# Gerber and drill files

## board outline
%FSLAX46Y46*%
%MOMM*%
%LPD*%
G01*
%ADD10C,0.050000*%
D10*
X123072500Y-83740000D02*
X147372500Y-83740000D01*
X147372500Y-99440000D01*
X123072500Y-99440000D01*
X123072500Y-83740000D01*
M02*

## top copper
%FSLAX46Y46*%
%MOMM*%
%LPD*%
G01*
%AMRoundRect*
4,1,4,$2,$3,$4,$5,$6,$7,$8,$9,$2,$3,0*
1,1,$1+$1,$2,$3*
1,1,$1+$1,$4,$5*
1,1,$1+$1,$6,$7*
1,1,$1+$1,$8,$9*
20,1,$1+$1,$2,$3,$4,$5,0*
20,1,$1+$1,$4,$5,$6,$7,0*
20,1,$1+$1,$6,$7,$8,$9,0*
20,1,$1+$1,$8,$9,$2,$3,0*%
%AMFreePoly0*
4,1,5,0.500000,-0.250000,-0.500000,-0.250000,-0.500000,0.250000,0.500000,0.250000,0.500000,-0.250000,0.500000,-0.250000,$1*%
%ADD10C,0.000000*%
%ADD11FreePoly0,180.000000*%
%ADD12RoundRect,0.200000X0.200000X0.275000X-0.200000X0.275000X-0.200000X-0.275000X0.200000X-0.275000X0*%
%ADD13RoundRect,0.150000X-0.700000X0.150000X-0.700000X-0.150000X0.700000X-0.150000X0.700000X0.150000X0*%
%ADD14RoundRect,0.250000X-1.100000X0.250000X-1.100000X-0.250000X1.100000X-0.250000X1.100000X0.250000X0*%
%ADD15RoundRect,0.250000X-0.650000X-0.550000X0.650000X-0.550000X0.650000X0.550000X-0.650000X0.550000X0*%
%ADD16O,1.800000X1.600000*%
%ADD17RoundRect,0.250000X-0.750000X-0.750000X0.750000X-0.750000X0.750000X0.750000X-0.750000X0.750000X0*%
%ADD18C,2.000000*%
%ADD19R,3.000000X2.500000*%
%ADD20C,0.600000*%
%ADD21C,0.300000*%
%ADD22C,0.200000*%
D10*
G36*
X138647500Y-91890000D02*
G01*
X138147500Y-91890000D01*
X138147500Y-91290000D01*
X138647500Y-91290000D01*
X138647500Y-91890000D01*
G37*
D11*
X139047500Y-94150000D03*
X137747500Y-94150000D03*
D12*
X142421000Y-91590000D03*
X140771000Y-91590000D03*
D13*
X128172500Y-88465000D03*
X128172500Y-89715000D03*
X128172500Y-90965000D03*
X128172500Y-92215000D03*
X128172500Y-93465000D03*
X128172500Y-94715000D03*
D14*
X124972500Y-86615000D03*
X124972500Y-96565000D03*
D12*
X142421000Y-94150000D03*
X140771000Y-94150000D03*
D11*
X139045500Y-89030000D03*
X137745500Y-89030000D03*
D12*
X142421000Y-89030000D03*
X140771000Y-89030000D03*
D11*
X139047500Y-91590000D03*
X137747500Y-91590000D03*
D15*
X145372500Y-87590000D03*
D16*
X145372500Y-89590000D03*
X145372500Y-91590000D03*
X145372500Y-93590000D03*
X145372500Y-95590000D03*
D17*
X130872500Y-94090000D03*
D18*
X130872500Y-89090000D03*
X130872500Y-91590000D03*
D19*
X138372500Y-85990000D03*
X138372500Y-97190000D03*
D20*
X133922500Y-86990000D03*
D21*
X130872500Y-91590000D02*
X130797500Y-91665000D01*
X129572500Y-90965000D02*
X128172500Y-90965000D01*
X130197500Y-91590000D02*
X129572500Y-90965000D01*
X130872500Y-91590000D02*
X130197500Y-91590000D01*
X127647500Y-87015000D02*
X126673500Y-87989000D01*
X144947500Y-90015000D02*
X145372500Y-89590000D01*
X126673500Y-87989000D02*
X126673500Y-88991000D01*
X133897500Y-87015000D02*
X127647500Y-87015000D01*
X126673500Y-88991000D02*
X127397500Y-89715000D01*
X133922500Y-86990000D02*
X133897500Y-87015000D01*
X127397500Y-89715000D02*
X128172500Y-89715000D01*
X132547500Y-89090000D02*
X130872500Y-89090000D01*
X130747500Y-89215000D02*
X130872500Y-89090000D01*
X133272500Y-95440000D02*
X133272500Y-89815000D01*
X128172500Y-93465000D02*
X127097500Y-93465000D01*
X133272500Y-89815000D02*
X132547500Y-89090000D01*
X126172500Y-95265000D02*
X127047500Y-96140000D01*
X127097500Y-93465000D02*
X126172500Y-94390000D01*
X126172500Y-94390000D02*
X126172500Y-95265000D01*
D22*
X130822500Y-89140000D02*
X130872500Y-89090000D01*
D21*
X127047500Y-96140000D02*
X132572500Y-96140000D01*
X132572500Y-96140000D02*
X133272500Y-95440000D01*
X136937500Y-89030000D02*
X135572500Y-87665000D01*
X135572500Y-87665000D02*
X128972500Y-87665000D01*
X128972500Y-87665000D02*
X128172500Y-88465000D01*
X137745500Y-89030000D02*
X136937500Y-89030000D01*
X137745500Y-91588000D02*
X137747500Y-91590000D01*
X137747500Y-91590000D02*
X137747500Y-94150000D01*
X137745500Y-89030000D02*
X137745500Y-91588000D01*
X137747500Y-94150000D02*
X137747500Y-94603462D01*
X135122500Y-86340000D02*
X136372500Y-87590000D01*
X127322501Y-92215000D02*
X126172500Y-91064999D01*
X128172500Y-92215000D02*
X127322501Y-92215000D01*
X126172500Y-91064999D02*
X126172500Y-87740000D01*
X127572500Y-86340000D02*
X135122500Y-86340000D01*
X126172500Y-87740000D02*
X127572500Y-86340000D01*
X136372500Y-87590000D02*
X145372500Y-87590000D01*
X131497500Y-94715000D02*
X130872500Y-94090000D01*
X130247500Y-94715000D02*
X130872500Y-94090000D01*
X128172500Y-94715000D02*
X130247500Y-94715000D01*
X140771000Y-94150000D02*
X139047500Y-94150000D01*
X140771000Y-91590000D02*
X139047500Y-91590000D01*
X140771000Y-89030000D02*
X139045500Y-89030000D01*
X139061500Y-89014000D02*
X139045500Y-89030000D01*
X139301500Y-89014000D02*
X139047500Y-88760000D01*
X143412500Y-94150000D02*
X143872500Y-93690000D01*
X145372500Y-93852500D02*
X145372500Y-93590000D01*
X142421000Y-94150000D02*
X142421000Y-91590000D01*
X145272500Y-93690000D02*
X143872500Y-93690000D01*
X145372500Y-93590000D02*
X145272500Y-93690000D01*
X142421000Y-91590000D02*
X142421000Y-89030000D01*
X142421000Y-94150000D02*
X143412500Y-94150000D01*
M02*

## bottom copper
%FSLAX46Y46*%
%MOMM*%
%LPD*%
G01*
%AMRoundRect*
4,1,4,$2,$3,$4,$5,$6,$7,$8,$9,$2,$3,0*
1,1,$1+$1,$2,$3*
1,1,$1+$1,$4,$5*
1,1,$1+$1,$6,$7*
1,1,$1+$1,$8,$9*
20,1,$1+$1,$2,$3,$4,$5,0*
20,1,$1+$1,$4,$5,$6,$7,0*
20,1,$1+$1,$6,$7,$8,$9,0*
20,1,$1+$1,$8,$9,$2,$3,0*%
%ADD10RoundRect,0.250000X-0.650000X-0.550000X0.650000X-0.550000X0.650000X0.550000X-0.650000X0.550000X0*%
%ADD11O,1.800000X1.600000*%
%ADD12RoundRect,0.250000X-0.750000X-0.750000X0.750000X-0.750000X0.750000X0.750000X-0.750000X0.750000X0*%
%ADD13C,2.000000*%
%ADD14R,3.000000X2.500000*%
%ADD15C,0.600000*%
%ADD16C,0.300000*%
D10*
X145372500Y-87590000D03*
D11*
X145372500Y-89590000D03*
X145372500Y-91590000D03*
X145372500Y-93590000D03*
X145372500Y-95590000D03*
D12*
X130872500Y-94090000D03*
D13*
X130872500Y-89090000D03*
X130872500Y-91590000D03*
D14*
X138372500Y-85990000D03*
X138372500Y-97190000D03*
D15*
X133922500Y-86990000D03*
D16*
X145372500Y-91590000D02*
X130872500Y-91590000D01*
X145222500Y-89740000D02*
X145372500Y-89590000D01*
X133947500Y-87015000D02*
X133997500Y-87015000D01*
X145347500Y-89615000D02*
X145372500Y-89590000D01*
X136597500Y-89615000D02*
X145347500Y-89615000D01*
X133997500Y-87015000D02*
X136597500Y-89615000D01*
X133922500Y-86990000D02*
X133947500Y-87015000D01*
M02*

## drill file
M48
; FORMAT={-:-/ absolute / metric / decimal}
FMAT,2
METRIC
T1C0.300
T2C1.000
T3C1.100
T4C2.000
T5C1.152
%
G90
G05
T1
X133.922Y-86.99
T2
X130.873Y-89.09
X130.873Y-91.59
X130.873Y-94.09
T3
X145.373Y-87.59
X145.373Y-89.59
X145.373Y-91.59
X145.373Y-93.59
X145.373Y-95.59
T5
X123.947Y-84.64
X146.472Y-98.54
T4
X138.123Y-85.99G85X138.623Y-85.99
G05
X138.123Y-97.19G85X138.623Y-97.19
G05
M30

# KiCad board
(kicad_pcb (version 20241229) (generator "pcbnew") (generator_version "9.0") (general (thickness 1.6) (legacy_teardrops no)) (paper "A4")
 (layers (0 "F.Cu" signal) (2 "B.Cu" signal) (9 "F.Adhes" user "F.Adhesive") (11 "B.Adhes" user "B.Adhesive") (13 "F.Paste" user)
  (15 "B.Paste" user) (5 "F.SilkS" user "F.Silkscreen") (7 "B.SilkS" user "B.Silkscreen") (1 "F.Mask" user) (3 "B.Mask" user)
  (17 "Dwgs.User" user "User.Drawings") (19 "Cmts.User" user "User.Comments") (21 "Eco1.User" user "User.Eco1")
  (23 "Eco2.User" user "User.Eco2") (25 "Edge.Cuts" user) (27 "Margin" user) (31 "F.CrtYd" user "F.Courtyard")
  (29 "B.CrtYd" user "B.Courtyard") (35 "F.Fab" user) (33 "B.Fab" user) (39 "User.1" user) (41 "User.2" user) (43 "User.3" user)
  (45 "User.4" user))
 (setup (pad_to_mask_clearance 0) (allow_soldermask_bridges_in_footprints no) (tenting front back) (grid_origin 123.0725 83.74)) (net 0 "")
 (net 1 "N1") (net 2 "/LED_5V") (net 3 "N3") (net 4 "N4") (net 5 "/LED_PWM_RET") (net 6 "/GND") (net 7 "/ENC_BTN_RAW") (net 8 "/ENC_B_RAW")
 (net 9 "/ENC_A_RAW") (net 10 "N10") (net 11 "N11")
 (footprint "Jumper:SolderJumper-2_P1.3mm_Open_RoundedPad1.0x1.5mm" (layer "F.Cu") (at 138.3975 94.15 180)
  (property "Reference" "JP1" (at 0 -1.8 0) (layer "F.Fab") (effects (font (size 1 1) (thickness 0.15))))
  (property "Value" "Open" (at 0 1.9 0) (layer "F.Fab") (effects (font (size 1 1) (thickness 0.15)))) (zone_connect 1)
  (pad "1" smd custom (at -0.65 0 180) (size 1 0.5) (layers "F.Cu" "F.Mask") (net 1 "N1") (zone_connect 2) (thermal_bridge_angle 45)
   (options (clearance outline) (anchor rect)) (primitives))
  (pad "2" smd custom (at 0.65 0 180) (size 1 0.5) (layers "F.Cu" "F.Mask") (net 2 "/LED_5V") (zone_connect 2) (thermal_bridge_angle 45)
   (options (clearance outline) (anchor rect)) (primitives)))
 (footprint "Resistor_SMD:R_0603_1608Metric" (layer "F.Cu") (at 141.596 91.59 180)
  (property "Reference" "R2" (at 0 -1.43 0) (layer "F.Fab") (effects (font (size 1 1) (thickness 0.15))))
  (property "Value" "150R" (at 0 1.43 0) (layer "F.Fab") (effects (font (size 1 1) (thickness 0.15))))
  (pad "1" smd roundrect (at -0.825 0 180) (size 0.8 0.95) (layers "F.Cu" "F.Mask" "F.Paste") (roundrect_rratio 0.25) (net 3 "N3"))
  (pad "2" smd roundrect (at 0.825 0 180) (size 0.8 0.95) (layers "F.Cu" "F.Mask" "F.Paste") (roundrect_rratio 0.25) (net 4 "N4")))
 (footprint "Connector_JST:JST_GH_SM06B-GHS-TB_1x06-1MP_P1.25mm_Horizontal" (layer "F.Cu") (at 126.3225 91.59 -90)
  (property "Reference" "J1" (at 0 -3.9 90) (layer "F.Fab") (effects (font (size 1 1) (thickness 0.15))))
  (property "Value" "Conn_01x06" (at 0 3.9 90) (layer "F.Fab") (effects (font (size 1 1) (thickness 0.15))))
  (pad "1" smd roundrect (at -3.125 -1.85 270) (size 0.6 1.7) (layers "F.Cu" "F.Mask" "F.Paste") (roundrect_rratio 0.25) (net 2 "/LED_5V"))
  (pad "2" smd roundrect (at -1.875 -1.85 270) (size 0.6 1.7) (layers "F.Cu" "F.Mask" "F.Paste") (roundrect_rratio 0.25)
   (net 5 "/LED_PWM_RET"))
  (pad "3" smd roundrect (at -0.625 -1.85 270) (size 0.6 1.7) (layers "F.Cu" "F.Mask" "F.Paste") (roundrect_rratio 0.25) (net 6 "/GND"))
  (pad "4" smd roundrect (at 0.625 -1.85 270) (size 0.6 1.7) (layers "F.Cu" "F.Mask" "F.Paste") (roundrect_rratio 0.25)
   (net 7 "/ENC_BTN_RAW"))
  (pad "5" smd roundrect (at 1.875 -1.85 270) (size 0.6 1.7) (layers "F.Cu" "F.Mask" "F.Paste") (roundrect_rratio 0.25) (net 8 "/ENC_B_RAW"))
  (pad "6" smd roundrect (at 3.125 -1.85 270) (size 0.6 1.7) (layers "F.Cu" "F.Mask" "F.Paste") (roundrect_rratio 0.25) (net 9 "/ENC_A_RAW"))
  (pad "MP" smd roundrect (at -4.975 1.35 270) (size 1 2.7) (layers "F.Cu" "F.Mask" "F.Paste") (roundrect_rratio 0.25))
  (pad "MP" smd roundrect (at 4.975 1.35 270) (size 1 2.7) (layers "F.Cu" "F.Mask" "F.Paste") (roundrect_rratio 0.25)))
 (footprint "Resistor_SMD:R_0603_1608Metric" (layer "F.Cu") (at 141.596 94.15 180)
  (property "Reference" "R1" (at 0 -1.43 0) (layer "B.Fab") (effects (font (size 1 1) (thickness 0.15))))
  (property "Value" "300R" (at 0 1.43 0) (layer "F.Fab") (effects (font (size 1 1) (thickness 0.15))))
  (pad "1" smd roundrect (at -0.825 0 180) (size 0.8 0.95) (layers "F.Cu" "F.Mask" "F.Paste") (roundrect_rratio 0.25) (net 3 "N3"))
  (pad "2" smd roundrect (at 0.825 0 180) (size 0.8 0.95) (layers "F.Cu" "F.Mask" "F.Paste") (roundrect_rratio 0.25) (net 1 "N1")))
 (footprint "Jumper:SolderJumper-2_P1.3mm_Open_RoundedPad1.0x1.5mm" (layer "F.Cu") (at 138.3955 89.03 180)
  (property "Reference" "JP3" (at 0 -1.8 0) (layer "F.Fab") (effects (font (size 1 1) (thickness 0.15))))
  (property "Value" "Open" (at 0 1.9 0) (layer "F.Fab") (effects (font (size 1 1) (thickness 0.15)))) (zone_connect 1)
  (pad "1" smd custom (at -0.65 0 180) (size 1 0.5) (layers "F.Cu" "F.Mask") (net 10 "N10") (zone_connect 2) (thermal_bridge_angle 45)
   (options (clearance outline) (anchor rect)) (primitives))
  (pad "2" smd custom (at 0.65 0 180) (size 1 0.5) (layers "F.Cu" "F.Mask") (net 2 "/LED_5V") (zone_connect 2) (thermal_bridge_angle 45)
   (options (clearance outline) (anchor rect)) (primitives)))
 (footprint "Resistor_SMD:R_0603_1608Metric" (layer "F.Cu") (at 141.596 89.03 180)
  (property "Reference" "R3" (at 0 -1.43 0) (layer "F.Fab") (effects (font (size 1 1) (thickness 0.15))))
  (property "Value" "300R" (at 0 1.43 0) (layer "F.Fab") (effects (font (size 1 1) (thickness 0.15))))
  (pad "1" smd roundrect (at -0.825 0 180) (size 0.8 0.95) (layers "F.Cu" "F.Mask" "F.Paste") (roundrect_rratio 0.25) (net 3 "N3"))
  (pad "2" smd roundrect (at 0.825 0 180) (size 0.8 0.95) (layers "F.Cu" "F.Mask" "F.Paste") (roundrect_rratio 0.25) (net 10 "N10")))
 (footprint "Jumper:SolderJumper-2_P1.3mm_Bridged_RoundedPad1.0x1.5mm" (layer "F.Cu") (at 138.3975 91.59 180)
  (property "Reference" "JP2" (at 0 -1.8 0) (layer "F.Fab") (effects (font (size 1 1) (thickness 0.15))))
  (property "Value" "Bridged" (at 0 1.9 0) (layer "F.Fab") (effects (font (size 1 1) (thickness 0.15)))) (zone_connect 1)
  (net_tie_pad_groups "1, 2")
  (fp_poly (pts (xy 0.25 -0.3) (xy -0.25 -0.3) (xy -0.25 0.3) (xy 0.25 0.3)) (stroke (width 0) (type solid)) (fill yes) (layer "F.Cu"))
  (pad "1" smd custom (at -0.65 0 180) (size 1 0.5) (layers "F.Cu" "F.Mask") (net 4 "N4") (zone_connect 2) (thermal_bridge_angle 45)
   (options (clearance outline) (anchor rect)) (primitives))
  (pad "2" smd custom (at 0.65 0 180) (size 1 0.5) (layers "F.Cu" "F.Mask") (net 2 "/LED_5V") (zone_connect 2) (thermal_bridge_angle 45)
   (options (clearance outline) (anchor rect)) (primitives)))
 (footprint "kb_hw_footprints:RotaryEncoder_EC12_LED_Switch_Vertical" (layer "B.Cu") (at 130.8725 94.09)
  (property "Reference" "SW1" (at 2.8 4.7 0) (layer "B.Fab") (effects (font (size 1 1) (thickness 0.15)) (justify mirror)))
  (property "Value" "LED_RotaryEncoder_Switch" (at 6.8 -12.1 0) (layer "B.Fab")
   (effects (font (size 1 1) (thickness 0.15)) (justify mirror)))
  (pad "1" thru_hole roundrect (at 14.5 -6.5) (size 1.8 1.6) (drill 1.1) (layers "*.Cu" "*.Mask") (remove_unused_layers no)
   (roundrect_rratio 0.15625) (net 7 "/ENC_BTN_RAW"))
  (pad "2" thru_hole oval (at 14.5 -4.5) (size 1.8 1.6) (drill 1.1) (layers "*.Cu" "*.Mask") (remove_unused_layers no)
   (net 5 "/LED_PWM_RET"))
  (pad "3" thru_hole oval (at 14.5 -2.5) (size 1.8 1.6) (drill 1.1) (layers "*.Cu" "*.Mask") (remove_unused_layers no) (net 6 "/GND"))
  (pad "4" thru_hole oval (at 14.5 -0.5) (size 1.8 1.6) (drill 1.1) (layers "*.Cu" "*.Mask") (remove_unused_layers no) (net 3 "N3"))
  (pad "5" thru_hole oval (at 14.5 1.5) (size 1.8 1.6) (drill 1.1) (layers "*.Cu" "*.Mask") (remove_unused_layers no) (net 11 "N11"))
  (pad "A" thru_hole roundrect (at 0 0) (size 2 2) (drill 1) (layers "*.Cu" "*.Mask") (remove_unused_layers no) (roundrect_rratio 0.125)
   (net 9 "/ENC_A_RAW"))
  (pad "B" thru_hole circle (at 0 -5) (size 2 2) (drill 1) (layers "*.Cu" "*.Mask") (remove_unused_layers no) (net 8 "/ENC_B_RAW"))
  (pad "C" thru_hole circle (at 0 -2.5) (size 2 2) (drill 1) (layers "*.Cu" "*.Mask") (remove_unused_layers no) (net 6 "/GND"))
  (pad "MP" thru_hole rect (at 7.5 -8.1) (size 3 2.5) (drill oval 2.5 2) (layers "*.Cu" "*.Mask") (remove_unused_layers no))
  (pad "MP" thru_hole rect (at 7.5 3.1) (size 3 2.5) (drill oval 2.5 2) (layers "*.Cu" "*.Mask") (remove_unused_layers no)))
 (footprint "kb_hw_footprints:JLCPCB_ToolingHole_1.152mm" (layer "B.Cu") (at 123.9475 84.64)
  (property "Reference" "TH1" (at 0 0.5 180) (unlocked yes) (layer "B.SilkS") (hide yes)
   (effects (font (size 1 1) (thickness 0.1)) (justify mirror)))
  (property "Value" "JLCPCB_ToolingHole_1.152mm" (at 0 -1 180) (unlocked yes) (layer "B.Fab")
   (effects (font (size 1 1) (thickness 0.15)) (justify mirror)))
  (pad "" np_thru_hole circle (at 0 0) (size 1.152 1.152) (drill 1.152) (layers "*.Cu" "*.Mask") (solder_mask_margin 0.148) (clearance 0.25)
   (thermal_bridge_angle 90)))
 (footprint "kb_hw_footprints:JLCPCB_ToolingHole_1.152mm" (layer "B.Cu") (at 146.4725 98.54)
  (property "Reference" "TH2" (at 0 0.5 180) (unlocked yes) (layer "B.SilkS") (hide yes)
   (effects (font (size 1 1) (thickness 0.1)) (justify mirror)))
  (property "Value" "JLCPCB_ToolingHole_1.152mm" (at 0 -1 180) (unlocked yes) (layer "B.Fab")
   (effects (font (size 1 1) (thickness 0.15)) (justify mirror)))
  (pad "" np_thru_hole circle (at 0 0) (size 1.152 1.152) (drill 1.152) (layers "*.Cu" "*.Mask") (solder_mask_margin 0.148) (clearance 0.25)
   (thermal_bridge_angle 90)))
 (gr_rect (start 123.0725 83.74) (end 147.3725 99.44) (stroke (width 0.05) (type solid)) (fill no) (layer "Edge.Cuts"))
 (segment (start 130.8725 91.59) (end 130.7975 91.665) (width 0.3) (layer "F.Cu") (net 6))
 (segment (start 129.5725 90.965) (end 128.1725 90.965) (width 0.3) (layer "F.Cu") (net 6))
 (segment (start 130.1975 91.59) (end 129.5725 90.965) (width 0.3) (layer "F.Cu") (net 6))
 (segment (start 130.8725 91.59) (end 130.1975 91.59) (width 0.3) (layer "F.Cu") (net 6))
 (segment (start 145.3725 91.59) (end 130.8725 91.59) (width 0.3) (layer "B.Cu") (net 6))
 (segment (start 127.6475 87.015) (end 126.6735 87.989) (width 0.3) (layer "F.Cu") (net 5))
 (segment (start 144.9475 90.015) (end 145.3725 89.59) (width 0.3) (layer "F.Cu") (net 5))
 (segment (start 126.6735 87.989) (end 126.6735 88.991) (width 0.3) (layer "F.Cu") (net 5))
 (segment (start 133.8975 87.015) (end 127.6475 87.015) (width 0.3) (layer "F.Cu") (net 5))
 (segment (start 126.6735 88.991) (end 127.3975 89.715) (width 0.3) (layer "F.Cu") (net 5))
 (segment (start 133.9225 86.99) (end 133.8975 87.015) (width 0.3) (layer "F.Cu") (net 5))
 (segment (start 127.3975 89.715) (end 128.1725 89.715) (width 0.3) (layer "F.Cu") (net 5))
 (via (at 133.9225 86.99) (size 0.6) (drill 0.3) (layers "F.Cu" "B.Cu") (free yes) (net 5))
 (segment (start 145.2225 89.74) (end 145.3725 89.59) (width 0.3) (layer "B.Cu") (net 5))
 (segment (start 133.9475 87.015) (end 133.9975 87.015) (width 0.3) (layer "B.Cu") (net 5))
 (segment (start 145.3475 89.615) (end 145.3725 89.59) (width 0.3) (layer "B.Cu") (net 5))
 (segment (start 136.5975 89.615) (end 145.3475 89.615) (width 0.3) (layer "B.Cu") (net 5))
 (segment (start 133.9975 87.015) (end 136.5975 89.615) (width 0.3) (layer "B.Cu") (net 5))
 (segment (start 133.9225 86.99) (end 133.9475 87.015) (width 0.3) (layer "B.Cu") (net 5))
 (segment (start 132.5475 89.09) (end 130.8725 89.09) (width 0.3) (layer "F.Cu") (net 8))
 (segment (start 130.7475 89.215) (end 130.8725 89.09) (width 0.3) (layer "F.Cu") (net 8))
 (segment (start 133.2725 95.44) (end 133.2725 89.815) (width 0.3) (layer "F.Cu") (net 8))
 (segment (start 128.1725 93.465) (end 127.0975 93.465) (width 0.3) (layer "F.Cu") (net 8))
 (segment (start 133.2725 89.815) (end 132.5475 89.09) (width 0.3) (layer "F.Cu") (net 8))
 (segment (start 126.1725 95.265) (end 127.0475 96.14) (width 0.3) (layer "F.Cu") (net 8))
 (segment (start 127.0975 93.465) (end 126.1725 94.39) (width 0.3) (layer "F.Cu") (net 8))
 (segment (start 126.1725 94.39) (end 126.1725 95.265) (width 0.3) (layer "F.Cu") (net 8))
 (segment (start 130.8225 89.14) (end 130.8725 89.09) (width 0.2) (layer "F.Cu") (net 8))
 (segment (start 127.0475 96.14) (end 132.5725 96.14) (width 0.3) (layer "F.Cu") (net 8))
 (segment (start 132.5725 96.14) (end 133.2725 95.44) (width 0.3) (layer "F.Cu") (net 8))
 (segment (start 136.9375 89.03) (end 135.5725 87.665) (width 0.3) (layer "F.Cu") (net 2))
 (segment (start 135.5725 87.665) (end 128.9725 87.665) (width 0.3) (layer "F.Cu") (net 2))
 (segment (start 128.9725 87.665) (end 128.1725 88.465) (width 0.3) (layer "F.Cu") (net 2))
 (segment (start 137.7455 89.03) (end 136.9375 89.03) (width 0.3) (layer "F.Cu") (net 2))
 (segment (start 137.7455 91.588) (end 137.7475 91.59) (width 0.3) (layer "F.Cu") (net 2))
 (segment (start 137.7475 91.59) (end 137.7475 94.15) (width 0.3) (layer "F.Cu") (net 2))
 (segment (start 137.7455 89.03) (end 137.7455 91.588) (width 0.3) (layer "F.Cu") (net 2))
 (segment (start 137.7475 94.15) (end 137.7475 94.603462) (width 0.3) (layer "F.Cu") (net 2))
 (segment (start 135.1225 86.34) (end 136.3725 87.59) (width 0.3) (layer "F.Cu") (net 7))
 (segment (start 127.322501 92.215) (end 126.1725 91.064999) (width 0.3) (layer "F.Cu") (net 7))
 (segment (start 128.1725 92.215) (end 127.322501 92.215) (width 0.3) (layer "F.Cu") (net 7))
 (segment (start 126.1725 91.064999) (end 126.1725 87.74) (width 0.3) (layer "F.Cu") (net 7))
 (segment (start 127.5725 86.34) (end 135.1225 86.34) (width 0.3) (layer "F.Cu") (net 7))
 (segment (start 126.1725 87.74) (end 127.5725 86.34) (width 0.3) (layer "F.Cu") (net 7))
 (segment (start 136.3725 87.59) (end 145.3725 87.59) (width 0.3) (layer "F.Cu") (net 7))
 (segment (start 131.4975 94.715) (end 130.8725 94.09) (width 0.3) (layer "F.Cu") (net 9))
 (segment (start 130.2475 94.715) (end 130.8725 94.09) (width 0.3) (layer "F.Cu") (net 9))
 (segment (start 128.1725 94.715) (end 130.2475 94.715) (width 0.3) (layer "F.Cu") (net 9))
 (segment (start 140.771 94.15) (end 139.0475 94.15) (width 0.3) (layer "F.Cu") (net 1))
 (segment (start 140.771 91.59) (end 139.0475 91.59) (width 0.3) (layer "F.Cu") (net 4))
 (segment (start 140.771 89.03) (end 139.0455 89.03) (width 0.3) (layer "F.Cu") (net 10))
 (segment (start 139.0615 89.014) (end 139.0455 89.03) (width 0.3) (layer "F.Cu") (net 10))
 (segment (start 139.3015 89.014) (end 139.0475 88.76) (width 0.3) (layer "F.Cu") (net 10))
 (segment (start 143.4125 94.15) (end 143.8725 93.69) (width 0.3) (layer "F.Cu") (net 3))
 (segment (start 145.3725 93.8525) (end 145.3725 93.59) (width 0.3) (layer "F.Cu") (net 3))
 (segment (start 142.421 94.15) (end 142.421 91.59) (width 0.3) (layer "F.Cu") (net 3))
 (segment (start 145.2725 93.69) (end 143.8725 93.69) (width 0.3) (layer "F.Cu") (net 3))
 (segment (start 145.3725 93.59) (end 145.2725 93.69) (width 0.3) (layer "F.Cu") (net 3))
 (segment (start 142.421 91.59) (end 142.421 89.03) (width 0.3) (layer "F.Cu") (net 3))
 (segment (start 142.421 94.15) (end 143.4125 94.15) (width 0.3) (layer "F.Cu") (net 3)))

